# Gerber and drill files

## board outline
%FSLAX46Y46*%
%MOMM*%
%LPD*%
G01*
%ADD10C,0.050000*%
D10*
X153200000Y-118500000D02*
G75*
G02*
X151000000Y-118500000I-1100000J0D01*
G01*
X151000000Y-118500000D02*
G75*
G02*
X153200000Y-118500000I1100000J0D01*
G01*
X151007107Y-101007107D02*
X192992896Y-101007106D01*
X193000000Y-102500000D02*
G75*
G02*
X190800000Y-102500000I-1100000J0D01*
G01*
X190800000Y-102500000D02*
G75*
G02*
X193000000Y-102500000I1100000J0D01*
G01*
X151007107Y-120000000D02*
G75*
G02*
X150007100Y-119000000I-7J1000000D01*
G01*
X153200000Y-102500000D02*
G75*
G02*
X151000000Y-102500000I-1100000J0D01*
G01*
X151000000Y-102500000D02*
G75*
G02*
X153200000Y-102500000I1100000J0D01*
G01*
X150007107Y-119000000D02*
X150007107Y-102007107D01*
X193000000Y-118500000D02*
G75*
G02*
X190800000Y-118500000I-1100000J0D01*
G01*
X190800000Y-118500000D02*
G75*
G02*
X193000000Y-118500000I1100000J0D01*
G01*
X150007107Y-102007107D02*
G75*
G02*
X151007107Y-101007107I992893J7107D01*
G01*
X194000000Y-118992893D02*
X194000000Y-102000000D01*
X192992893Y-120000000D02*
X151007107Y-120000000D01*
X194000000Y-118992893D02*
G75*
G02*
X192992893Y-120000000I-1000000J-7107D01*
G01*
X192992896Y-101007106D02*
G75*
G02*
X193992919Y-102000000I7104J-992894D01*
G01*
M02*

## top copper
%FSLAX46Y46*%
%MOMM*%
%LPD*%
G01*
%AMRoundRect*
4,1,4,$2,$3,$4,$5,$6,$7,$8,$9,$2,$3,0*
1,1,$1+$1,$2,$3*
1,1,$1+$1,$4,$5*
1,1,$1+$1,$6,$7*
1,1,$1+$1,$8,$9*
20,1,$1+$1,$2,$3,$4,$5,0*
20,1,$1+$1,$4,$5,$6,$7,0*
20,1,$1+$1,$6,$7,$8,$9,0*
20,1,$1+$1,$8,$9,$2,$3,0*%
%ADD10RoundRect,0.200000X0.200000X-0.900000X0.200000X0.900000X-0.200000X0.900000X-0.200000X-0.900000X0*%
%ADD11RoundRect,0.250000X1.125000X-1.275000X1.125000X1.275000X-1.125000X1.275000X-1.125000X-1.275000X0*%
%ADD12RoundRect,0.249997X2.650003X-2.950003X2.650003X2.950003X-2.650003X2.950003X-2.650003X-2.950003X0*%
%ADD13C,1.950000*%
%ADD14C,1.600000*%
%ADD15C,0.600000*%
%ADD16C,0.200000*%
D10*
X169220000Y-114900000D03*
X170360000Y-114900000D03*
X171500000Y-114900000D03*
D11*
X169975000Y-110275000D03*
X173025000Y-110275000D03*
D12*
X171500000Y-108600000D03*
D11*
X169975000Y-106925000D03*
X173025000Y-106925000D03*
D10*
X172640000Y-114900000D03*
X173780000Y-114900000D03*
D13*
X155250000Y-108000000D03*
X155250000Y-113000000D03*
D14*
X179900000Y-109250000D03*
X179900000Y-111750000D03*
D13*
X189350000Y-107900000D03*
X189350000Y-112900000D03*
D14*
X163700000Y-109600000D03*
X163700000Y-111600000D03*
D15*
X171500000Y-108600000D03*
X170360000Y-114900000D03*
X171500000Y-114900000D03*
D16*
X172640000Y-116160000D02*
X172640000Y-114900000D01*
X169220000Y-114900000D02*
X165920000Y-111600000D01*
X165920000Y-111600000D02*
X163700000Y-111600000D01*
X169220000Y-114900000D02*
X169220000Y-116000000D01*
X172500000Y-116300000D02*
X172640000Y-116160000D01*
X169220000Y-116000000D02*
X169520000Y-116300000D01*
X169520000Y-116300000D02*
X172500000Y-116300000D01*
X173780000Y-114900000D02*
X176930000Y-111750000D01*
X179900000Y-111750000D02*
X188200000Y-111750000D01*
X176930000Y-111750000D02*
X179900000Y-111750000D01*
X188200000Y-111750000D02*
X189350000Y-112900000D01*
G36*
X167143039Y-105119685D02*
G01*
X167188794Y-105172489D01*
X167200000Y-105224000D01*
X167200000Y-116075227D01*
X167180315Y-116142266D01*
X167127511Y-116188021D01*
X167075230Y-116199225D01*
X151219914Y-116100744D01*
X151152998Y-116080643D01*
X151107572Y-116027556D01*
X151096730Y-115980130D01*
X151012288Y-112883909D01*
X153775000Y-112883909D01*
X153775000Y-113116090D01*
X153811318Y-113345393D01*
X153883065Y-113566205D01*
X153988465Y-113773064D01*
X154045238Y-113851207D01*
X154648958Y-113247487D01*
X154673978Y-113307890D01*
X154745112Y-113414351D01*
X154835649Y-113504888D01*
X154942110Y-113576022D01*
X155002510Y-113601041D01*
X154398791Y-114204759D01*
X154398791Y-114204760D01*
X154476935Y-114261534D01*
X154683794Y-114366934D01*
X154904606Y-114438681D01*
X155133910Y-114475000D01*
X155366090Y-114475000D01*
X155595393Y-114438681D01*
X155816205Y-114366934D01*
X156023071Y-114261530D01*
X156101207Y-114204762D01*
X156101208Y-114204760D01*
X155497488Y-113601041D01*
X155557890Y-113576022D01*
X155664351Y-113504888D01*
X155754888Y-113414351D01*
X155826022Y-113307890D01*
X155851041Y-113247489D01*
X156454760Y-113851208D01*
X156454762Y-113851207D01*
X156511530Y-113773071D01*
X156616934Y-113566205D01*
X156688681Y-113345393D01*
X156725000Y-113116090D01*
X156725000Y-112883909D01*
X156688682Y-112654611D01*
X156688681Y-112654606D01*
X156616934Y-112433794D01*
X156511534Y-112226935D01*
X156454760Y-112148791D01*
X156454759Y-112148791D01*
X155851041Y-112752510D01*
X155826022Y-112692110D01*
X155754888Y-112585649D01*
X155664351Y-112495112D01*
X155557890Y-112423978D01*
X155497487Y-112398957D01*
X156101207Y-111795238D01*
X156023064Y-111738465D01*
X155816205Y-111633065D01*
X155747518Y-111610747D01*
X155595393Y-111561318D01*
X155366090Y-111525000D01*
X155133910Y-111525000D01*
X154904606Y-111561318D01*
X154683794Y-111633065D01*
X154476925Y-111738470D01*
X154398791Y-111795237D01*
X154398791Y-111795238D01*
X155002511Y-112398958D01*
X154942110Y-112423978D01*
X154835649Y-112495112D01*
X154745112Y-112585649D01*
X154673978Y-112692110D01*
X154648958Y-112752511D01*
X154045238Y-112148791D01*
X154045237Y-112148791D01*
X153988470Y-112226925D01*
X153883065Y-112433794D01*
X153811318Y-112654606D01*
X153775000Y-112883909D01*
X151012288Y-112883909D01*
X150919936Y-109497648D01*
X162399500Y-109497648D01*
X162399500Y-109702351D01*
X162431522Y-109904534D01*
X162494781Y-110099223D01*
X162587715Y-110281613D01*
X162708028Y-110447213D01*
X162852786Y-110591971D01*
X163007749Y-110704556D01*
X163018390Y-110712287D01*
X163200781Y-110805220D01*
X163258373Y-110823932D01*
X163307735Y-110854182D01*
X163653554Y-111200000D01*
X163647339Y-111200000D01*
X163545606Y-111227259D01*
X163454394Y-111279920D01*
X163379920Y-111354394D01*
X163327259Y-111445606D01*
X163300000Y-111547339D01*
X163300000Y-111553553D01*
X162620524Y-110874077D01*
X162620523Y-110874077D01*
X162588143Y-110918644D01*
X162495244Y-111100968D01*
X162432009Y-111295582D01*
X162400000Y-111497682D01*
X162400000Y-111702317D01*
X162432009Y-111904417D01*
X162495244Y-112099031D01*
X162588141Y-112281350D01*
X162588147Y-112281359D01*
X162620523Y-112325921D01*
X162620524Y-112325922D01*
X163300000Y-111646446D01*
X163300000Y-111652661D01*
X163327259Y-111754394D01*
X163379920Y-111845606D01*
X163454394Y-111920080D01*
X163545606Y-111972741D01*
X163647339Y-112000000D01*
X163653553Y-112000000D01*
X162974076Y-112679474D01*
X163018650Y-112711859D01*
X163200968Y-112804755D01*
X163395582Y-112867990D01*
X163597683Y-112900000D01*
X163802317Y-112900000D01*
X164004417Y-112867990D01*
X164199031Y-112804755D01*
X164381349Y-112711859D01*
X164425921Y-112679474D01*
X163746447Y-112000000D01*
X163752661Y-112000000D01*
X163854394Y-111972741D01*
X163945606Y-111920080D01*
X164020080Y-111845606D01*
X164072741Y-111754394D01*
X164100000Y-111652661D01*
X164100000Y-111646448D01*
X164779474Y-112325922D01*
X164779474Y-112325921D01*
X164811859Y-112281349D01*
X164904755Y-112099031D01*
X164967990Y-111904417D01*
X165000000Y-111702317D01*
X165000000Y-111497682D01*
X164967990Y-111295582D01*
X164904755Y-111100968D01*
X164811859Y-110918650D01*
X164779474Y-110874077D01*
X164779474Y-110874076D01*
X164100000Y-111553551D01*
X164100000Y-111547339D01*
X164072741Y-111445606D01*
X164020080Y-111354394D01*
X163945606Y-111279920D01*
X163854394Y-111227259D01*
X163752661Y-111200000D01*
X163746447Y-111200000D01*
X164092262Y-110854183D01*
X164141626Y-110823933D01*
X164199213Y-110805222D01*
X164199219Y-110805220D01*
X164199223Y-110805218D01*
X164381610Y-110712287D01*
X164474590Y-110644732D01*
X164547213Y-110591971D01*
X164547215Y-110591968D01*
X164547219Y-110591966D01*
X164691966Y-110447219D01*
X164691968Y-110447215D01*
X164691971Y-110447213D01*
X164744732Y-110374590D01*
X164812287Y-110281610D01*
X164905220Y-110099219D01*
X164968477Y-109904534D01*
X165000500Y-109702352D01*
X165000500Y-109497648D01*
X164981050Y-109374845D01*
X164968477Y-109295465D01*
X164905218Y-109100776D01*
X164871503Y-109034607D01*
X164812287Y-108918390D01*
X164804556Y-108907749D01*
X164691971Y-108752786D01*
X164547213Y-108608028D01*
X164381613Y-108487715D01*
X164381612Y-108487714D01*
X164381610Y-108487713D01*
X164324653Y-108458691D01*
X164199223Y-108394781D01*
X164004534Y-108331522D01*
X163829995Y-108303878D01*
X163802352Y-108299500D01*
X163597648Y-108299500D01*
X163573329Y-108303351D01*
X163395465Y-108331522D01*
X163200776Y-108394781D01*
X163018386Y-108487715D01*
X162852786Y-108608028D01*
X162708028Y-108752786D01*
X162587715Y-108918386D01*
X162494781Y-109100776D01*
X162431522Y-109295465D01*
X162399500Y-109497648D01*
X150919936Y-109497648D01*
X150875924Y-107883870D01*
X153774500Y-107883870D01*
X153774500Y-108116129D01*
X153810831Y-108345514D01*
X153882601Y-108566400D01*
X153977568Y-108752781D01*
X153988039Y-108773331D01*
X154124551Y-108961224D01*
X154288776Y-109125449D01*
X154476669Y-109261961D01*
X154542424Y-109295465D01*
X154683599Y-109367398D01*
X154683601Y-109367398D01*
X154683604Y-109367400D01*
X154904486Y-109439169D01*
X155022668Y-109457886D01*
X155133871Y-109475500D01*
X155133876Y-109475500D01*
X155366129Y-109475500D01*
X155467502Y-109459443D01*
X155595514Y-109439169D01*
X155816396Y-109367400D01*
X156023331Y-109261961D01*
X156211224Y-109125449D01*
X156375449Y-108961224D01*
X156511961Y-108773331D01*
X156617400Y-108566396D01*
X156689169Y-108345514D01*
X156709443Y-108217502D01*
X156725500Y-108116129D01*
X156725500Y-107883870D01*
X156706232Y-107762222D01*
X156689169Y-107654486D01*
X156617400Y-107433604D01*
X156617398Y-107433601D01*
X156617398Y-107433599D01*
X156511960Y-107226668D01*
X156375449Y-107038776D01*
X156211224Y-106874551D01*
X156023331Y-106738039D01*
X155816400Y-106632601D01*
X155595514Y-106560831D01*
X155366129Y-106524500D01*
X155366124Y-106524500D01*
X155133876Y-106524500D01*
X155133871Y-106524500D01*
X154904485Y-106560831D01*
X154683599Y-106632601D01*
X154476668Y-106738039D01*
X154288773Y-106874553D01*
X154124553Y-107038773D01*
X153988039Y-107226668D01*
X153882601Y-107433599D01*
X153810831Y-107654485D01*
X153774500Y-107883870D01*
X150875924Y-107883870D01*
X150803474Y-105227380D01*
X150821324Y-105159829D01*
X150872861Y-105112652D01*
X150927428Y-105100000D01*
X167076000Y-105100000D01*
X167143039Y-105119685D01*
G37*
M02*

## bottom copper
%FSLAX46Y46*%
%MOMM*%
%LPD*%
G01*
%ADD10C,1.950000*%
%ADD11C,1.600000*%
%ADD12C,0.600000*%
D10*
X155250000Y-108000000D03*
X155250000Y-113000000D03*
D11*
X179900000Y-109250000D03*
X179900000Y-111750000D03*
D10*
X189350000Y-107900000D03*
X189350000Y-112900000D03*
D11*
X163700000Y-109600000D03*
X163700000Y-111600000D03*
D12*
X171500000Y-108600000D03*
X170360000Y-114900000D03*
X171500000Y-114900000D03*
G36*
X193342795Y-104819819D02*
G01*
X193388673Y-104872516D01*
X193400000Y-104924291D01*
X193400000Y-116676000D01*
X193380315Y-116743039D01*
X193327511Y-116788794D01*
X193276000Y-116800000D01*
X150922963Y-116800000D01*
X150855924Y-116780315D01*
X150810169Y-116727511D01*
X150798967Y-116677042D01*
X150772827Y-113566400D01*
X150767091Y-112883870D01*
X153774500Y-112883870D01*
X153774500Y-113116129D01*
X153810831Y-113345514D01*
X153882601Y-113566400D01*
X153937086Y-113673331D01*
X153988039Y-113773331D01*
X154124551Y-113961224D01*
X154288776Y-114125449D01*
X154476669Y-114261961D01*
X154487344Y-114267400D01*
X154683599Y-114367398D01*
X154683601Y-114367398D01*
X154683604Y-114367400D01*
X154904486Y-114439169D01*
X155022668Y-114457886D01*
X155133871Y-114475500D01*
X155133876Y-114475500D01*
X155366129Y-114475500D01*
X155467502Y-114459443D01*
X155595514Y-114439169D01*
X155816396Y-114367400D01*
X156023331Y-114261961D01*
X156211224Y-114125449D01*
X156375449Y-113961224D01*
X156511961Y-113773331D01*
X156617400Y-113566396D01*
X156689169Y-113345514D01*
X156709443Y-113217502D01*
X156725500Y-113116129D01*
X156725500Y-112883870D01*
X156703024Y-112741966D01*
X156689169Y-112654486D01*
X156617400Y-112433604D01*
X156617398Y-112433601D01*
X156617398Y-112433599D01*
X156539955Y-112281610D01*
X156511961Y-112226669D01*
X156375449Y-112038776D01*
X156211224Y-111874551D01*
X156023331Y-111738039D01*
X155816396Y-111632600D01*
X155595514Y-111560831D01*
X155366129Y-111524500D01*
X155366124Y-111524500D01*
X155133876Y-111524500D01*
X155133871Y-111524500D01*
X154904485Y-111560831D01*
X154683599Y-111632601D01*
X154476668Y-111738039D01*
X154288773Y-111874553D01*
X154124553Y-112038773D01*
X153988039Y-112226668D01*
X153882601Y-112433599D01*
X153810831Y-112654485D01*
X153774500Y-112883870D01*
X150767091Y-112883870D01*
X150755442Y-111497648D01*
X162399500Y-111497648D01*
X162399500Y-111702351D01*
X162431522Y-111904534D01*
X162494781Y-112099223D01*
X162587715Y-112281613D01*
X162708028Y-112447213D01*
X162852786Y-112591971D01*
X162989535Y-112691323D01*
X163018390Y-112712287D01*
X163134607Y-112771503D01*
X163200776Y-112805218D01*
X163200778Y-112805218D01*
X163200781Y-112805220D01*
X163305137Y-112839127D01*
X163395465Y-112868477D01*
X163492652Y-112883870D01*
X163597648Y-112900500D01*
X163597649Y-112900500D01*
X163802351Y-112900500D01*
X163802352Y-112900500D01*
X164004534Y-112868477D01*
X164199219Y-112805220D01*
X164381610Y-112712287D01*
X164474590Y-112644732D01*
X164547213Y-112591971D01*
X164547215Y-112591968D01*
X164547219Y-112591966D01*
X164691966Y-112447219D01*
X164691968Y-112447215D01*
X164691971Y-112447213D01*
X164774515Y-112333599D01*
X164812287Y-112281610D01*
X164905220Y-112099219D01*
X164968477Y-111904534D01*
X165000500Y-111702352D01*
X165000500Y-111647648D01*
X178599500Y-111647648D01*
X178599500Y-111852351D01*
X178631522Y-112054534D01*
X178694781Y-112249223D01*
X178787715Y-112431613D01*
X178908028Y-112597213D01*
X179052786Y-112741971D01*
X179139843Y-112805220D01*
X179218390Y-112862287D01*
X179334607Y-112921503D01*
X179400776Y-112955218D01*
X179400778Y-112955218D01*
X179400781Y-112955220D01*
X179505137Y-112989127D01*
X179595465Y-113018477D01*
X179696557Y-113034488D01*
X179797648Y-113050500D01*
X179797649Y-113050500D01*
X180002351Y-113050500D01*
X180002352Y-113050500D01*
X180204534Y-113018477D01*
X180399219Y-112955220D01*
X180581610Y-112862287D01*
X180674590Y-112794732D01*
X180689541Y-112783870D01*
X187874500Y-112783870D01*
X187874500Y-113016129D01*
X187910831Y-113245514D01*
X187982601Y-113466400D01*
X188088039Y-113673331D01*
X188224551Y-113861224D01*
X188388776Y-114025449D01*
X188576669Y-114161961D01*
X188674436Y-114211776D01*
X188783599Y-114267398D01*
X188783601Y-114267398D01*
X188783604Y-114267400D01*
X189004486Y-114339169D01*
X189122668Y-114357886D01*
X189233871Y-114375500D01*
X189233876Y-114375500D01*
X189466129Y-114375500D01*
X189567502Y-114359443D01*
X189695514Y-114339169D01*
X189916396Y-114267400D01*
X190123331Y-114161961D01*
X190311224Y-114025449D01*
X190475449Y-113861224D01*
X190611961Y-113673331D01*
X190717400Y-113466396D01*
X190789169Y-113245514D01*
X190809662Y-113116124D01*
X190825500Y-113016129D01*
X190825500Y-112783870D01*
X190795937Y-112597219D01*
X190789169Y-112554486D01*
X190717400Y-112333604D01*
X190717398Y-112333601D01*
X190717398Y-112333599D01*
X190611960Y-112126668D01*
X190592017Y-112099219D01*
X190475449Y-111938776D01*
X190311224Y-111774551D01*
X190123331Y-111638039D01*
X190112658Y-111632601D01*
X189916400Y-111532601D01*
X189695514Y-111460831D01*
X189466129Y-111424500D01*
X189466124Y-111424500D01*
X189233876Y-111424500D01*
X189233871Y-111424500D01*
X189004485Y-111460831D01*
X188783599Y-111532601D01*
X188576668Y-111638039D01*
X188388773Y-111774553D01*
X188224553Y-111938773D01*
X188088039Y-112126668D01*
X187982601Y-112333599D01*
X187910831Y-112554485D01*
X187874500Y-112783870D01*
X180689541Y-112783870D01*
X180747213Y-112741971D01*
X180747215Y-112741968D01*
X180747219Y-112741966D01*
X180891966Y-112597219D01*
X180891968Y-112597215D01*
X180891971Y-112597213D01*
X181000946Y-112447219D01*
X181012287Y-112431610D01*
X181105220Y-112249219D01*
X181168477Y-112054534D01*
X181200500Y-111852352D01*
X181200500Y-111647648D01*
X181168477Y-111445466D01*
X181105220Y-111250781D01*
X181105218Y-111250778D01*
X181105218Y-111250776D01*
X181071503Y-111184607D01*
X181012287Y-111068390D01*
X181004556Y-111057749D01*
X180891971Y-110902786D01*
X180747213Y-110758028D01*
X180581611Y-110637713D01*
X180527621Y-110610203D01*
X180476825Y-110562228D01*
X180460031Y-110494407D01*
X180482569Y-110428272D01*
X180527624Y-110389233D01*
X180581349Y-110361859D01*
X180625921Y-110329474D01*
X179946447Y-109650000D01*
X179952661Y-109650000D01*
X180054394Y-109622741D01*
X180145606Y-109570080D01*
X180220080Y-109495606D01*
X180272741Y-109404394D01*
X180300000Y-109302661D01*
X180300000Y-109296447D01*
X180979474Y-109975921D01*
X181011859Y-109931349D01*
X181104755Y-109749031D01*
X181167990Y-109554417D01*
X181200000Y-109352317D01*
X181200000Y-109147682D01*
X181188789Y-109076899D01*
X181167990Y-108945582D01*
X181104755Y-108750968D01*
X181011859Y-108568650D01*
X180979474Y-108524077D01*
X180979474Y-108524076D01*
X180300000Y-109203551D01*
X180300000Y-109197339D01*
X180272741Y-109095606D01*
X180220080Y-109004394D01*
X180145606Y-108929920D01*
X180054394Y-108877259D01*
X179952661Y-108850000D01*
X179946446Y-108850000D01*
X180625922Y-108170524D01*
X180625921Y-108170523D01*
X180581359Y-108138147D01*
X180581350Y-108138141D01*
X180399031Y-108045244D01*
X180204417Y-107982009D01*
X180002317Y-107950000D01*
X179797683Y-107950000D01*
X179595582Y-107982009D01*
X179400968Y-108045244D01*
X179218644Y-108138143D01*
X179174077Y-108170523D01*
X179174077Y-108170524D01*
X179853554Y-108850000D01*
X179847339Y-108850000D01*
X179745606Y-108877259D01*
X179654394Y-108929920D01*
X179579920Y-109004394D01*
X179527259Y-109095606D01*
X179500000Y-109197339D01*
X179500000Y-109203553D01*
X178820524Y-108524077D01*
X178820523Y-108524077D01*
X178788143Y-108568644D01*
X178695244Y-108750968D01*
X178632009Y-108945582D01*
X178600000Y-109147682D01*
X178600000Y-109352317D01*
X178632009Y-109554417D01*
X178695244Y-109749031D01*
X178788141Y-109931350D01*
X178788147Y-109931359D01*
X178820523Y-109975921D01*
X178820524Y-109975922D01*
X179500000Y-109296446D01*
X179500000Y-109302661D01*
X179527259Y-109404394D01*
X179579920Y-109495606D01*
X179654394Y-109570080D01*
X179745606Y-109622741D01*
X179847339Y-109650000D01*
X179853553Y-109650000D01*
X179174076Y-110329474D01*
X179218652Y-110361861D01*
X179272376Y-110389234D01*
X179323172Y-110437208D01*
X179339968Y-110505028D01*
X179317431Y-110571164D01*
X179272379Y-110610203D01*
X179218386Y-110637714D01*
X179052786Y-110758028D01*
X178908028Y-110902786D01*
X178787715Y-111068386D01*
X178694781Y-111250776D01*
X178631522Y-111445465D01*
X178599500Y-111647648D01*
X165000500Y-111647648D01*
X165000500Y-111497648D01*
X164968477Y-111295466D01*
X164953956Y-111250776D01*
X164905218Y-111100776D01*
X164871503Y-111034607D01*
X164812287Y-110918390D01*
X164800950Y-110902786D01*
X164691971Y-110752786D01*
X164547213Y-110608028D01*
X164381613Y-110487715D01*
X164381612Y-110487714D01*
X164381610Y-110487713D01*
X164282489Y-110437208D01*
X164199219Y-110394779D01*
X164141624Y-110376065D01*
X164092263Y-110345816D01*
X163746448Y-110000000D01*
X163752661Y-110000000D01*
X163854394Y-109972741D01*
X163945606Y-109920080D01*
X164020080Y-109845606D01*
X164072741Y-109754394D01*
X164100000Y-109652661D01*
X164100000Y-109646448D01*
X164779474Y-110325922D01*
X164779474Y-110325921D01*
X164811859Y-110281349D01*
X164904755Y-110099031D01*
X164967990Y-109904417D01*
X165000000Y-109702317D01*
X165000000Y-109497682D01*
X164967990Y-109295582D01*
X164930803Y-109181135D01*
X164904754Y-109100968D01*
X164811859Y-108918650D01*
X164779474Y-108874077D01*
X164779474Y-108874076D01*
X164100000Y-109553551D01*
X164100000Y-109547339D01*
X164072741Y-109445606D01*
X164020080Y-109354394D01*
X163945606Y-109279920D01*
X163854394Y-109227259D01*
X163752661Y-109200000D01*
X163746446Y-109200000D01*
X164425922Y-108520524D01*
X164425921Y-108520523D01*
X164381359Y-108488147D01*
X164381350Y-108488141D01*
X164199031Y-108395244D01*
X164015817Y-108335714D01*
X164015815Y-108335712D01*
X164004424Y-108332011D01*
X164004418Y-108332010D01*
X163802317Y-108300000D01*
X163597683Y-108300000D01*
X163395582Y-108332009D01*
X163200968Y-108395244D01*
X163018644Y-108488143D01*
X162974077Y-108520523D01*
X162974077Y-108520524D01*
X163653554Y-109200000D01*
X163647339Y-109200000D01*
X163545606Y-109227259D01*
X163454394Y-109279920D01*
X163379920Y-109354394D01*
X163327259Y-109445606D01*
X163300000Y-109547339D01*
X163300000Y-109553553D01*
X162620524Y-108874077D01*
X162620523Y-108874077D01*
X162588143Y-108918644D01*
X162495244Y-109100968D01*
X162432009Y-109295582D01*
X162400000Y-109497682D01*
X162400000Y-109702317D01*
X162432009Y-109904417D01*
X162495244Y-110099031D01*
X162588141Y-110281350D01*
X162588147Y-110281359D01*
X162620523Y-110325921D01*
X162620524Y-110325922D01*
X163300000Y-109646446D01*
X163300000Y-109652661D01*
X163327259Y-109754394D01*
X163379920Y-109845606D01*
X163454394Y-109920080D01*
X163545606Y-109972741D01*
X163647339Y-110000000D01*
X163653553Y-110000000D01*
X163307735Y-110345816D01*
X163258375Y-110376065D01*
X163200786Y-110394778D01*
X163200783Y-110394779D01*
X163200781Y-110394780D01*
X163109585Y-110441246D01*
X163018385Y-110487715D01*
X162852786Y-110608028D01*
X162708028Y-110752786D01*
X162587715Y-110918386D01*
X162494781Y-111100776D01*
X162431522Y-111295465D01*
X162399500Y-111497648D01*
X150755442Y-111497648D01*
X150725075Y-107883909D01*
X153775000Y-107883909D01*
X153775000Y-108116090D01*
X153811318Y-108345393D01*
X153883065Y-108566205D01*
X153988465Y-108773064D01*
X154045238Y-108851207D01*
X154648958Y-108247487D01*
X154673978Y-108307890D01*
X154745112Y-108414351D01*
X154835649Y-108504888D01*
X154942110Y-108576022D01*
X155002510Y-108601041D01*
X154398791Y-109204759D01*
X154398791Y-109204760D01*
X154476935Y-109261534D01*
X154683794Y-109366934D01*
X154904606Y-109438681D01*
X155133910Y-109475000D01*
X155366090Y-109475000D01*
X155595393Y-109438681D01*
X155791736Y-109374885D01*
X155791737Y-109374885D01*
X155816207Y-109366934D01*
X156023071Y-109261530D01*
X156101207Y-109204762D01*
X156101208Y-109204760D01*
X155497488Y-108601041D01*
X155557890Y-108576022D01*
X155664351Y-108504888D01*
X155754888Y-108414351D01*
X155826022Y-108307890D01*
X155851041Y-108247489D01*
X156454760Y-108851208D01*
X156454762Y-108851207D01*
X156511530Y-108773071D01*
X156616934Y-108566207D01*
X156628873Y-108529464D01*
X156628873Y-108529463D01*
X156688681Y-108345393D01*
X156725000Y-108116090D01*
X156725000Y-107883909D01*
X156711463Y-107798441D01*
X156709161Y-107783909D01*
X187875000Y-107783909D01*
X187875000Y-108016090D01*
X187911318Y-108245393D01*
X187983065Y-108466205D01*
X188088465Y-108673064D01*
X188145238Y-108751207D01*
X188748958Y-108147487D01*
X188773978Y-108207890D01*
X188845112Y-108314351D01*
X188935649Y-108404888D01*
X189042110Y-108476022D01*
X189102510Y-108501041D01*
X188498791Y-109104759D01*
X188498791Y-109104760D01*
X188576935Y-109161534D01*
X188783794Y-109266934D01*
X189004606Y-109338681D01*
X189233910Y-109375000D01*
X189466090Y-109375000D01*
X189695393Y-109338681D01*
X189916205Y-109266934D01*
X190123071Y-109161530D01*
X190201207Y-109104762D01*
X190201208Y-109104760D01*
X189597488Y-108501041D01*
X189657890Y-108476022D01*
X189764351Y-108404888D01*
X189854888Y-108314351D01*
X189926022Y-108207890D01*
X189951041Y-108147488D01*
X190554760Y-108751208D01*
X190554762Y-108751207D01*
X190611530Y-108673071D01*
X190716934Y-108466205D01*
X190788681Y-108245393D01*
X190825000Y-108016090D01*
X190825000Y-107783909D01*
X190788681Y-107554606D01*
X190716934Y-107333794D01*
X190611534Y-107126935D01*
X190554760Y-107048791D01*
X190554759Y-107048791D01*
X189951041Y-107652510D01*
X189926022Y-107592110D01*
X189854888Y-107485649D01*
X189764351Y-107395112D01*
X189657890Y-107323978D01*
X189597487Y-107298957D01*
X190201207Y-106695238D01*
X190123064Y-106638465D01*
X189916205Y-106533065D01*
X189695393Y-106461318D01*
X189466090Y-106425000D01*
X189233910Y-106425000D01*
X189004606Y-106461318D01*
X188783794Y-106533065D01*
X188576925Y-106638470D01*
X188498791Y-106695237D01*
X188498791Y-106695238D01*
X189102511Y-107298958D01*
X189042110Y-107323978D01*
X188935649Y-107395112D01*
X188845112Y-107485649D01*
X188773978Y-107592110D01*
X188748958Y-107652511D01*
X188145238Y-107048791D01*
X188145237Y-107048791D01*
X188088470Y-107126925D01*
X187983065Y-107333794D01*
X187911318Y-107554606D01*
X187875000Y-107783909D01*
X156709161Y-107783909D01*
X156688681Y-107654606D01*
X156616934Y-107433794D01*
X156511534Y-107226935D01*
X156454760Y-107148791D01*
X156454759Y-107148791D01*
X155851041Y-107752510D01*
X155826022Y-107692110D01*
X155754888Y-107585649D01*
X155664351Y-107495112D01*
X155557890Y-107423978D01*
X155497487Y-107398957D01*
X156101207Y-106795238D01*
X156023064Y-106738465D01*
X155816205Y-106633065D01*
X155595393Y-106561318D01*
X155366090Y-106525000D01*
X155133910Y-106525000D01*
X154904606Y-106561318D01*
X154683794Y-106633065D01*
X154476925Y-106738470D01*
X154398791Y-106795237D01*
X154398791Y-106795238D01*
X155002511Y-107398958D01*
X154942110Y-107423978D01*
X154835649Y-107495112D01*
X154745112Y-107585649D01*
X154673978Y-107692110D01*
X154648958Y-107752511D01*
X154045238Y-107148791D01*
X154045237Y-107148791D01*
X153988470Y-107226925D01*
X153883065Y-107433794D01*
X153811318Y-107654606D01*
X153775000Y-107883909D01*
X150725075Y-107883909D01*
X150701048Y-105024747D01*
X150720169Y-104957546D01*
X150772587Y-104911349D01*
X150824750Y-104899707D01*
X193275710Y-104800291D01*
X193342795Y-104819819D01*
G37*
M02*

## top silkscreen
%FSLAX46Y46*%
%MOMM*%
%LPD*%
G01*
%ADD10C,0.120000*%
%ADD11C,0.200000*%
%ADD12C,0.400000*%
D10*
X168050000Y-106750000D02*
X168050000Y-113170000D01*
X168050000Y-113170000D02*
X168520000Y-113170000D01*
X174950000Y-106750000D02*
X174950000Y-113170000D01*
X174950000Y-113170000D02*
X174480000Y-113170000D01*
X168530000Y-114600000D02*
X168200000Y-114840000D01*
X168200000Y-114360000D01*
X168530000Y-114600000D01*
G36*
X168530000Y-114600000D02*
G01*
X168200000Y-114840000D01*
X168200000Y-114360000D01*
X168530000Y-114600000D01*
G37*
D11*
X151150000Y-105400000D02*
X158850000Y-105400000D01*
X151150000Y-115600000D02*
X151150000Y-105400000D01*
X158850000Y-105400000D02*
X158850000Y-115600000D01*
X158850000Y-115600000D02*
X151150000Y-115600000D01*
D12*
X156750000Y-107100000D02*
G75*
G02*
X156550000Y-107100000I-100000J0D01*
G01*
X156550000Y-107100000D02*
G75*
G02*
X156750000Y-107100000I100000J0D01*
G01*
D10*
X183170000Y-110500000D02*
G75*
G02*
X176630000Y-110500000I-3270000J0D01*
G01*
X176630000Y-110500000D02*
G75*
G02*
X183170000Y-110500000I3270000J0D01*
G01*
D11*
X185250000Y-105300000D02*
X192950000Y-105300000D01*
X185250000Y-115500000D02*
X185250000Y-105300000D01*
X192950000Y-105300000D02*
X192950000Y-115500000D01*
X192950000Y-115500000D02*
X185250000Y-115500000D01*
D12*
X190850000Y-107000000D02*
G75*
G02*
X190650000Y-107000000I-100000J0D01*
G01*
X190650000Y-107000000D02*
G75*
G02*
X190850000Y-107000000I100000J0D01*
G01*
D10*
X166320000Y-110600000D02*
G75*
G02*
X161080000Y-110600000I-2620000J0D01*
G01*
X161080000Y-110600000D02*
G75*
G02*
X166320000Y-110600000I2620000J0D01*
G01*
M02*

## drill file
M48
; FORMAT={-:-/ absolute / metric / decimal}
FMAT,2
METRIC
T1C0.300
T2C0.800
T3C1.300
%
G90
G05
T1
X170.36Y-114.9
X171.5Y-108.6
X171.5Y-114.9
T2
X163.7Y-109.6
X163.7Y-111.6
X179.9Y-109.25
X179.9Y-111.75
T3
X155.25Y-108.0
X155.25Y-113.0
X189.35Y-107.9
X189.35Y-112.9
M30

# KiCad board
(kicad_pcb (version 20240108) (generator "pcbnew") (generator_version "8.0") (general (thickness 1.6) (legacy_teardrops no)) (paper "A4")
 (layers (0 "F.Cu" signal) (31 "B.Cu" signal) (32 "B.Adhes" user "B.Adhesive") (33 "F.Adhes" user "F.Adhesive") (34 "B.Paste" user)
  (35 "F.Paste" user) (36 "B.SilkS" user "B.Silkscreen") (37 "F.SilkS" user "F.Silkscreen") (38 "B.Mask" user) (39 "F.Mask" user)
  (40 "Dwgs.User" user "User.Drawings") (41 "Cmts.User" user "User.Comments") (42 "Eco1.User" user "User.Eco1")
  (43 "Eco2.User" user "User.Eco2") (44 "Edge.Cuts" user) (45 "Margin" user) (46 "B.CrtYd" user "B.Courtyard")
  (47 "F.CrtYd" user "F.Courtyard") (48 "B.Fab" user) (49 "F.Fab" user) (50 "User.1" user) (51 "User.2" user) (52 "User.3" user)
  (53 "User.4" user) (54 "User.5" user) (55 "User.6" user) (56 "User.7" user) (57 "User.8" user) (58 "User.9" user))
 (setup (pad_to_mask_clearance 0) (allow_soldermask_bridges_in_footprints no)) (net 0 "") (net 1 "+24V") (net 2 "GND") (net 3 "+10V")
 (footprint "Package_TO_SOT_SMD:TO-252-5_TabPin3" (layer "F.Cu") (at 171.5 109.86 90)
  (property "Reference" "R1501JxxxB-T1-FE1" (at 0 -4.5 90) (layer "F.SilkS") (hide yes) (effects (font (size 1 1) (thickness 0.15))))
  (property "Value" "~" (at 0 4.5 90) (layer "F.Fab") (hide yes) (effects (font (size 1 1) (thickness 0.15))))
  (fp_line (start 3.11 -3.45) (end -3.31 -3.45) (stroke (width 0.12) (type solid)) (layer "F.SilkS"))
  (fp_line (start -3.31 -3.45) (end -3.31 -2.98) (stroke (width 0.12) (type solid)) (layer "F.SilkS"))
  (fp_line (start 3.11 3.45) (end -3.31 3.45) (stroke (width 0.12) (type solid)) (layer "F.SilkS"))
  (fp_line (start -3.31 3.45) (end -3.31 2.98) (stroke (width 0.12) (type solid)) (layer "F.SilkS"))
  (fp_poly
   (pts (xy -4.74 -2.97) (xy -4.98 -3.3) (xy -4.5 -3.3) (xy -4.74 -2.97)) (stroke (width 0.12) (type solid)) (fill solid) (layer "F.SilkS"))
  (pad "1" smd roundrect (at -5.04 -2.28 90) (size 2.2 0.8) (layers "F.Cu" "F.Paste" "F.Mask") (roundrect_rratio 0.25) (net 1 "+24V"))
  (pad "2" smd roundrect (at -5.04 -1.14 90) (size 2.2 0.8) (layers "F.Cu" "F.Paste" "F.Mask") (roundrect_rratio 0.25) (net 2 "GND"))
  (pad "3" smd roundrect (at -5.04 0 90) (size 2.2 0.8) (layers "F.Cu" "F.Paste" "F.Mask") (roundrect_rratio 0.25) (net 2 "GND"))
  (pad "3" smd roundrect (at -0.415 -1.525 90) (size 3.05 2.75) (layers "F.Cu" "F.Paste") (roundrect_rratio 0.090909) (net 2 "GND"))
  (pad "3" smd roundrect (at -0.415 1.525 90) (size 3.05 2.75) (layers "F.Cu" "F.Paste") (roundrect_rratio 0.090909) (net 2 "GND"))
  (pad "3" smd roundrect (at 1.26 0 90) (size 6.4 5.8) (layers "F.Cu" "F.Mask") (roundrect_rratio 0.043103) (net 2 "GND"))
  (pad "3" smd roundrect (at 2.935 -1.525 90) (size 3.05 2.75) (layers "F.Cu" "F.Paste") (roundrect_rratio 0.090909) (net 2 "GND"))
  (pad "3" smd roundrect (at 2.935 1.525 90) (size 3.05 2.75) (layers "F.Cu" "F.Paste") (roundrect_rratio 0.090909) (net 2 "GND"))
  (pad "4" smd roundrect (at -5.04 1.14 90) (size 2.2 0.8) (layers "F.Cu" "F.Paste" "F.Mask") (roundrect_rratio 0.25) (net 1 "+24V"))
  (pad "5" smd roundrect (at -5.04 2.28 90) (size 2.2 0.8) (layers "F.Cu" "F.Paste" "F.Mask") (roundrect_rratio 0.25) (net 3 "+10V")))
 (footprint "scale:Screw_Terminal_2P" (layer "F.Cu") (at 155.25 110.5 -90)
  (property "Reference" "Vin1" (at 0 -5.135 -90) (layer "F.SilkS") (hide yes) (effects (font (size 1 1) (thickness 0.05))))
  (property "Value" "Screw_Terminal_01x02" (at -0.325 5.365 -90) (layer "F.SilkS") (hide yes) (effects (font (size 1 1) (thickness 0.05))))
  (fp_line (start -5.1 4.1) (end -5.1 -3.6) (stroke (width 0.2) (type solid)) (layer "F.SilkS"))
  (fp_line (start 5.1 4.1) (end -5.1 4.1) (stroke (width 0.2) (type solid)) (layer "F.SilkS"))
  (fp_line (start -5.1 -3.6) (end 5.1 -3.6) (stroke (width 0.2) (type solid)) (layer "F.SilkS"))
  (fp_line (start 5.1 -3.6) (end 5.1 4.1) (stroke (width 0.2) (type solid)) (layer "F.SilkS"))
  (fp_circle (center -3.4 -1.4) (end -3.3 -1.4) (stroke (width 0.4) (type solid)) (fill none) (layer "F.SilkS"))
  (pad "1" thru_hole circle (at -2.5 0 270) (size 1.95 1.95) (drill 1.3) (layers "*.Cu" "*.Mask") (remove_unused_layers no) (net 2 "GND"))
  (pad "2" thru_hole circle (at 2.5 0 270) (size 1.95 1.95) (drill 1.3) (layers "*.Cu" "*.Mask") (remove_unused_layers no) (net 1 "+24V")))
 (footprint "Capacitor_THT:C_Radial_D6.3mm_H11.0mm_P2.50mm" (layer "F.Cu") (at 179.9 109.25 -90)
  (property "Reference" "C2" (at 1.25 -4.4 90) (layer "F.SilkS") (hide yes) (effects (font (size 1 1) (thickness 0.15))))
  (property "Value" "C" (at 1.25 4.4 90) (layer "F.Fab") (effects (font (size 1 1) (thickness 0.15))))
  (fp_circle (center 1.25 0) (end 4.52 0) (stroke (width 0.12) (type solid)) (fill none) (layer "F.SilkS"))
  (pad "1" thru_hole circle (at 0 0 270) (size 1.6 1.6) (drill 0.8) (layers "*.Cu" "*.Mask") (remove_unused_layers no) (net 2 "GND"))
  (pad "2" thru_hole circle (at 2.5 0 270) (size 1.6 1.6) (drill 0.8) (layers "*.Cu" "*.Mask") (remove_unused_layers no) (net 3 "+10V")))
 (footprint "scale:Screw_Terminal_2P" (layer "F.Cu") (at 189.35 110.4 -90)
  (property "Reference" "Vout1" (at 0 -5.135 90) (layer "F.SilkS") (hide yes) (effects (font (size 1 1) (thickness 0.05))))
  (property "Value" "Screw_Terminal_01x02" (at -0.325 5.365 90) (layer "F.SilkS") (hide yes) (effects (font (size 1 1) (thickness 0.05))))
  (fp_line (start -5.1 4.1) (end -5.1 -3.6) (stroke (width 0.2) (type solid)) (layer "F.SilkS"))
  (fp_line (start 5.1 4.1) (end -5.1 4.1) (stroke (width 0.2) (type solid)) (layer "F.SilkS"))
  (fp_line (start -5.1 -3.6) (end 5.1 -3.6) (stroke (width 0.2) (type solid)) (layer "F.SilkS"))
  (fp_line (start 5.1 -3.6) (end 5.1 4.1) (stroke (width 0.2) (type solid)) (layer "F.SilkS"))
  (fp_circle (center -3.4 -1.4) (end -3.3 -1.4) (stroke (width 0.4) (type solid)) (fill none) (layer "F.SilkS"))
  (pad "1" thru_hole circle (at -2.5 0 270) (size 1.95 1.95) (drill 1.3) (layers "*.Cu" "*.Mask") (remove_unused_layers no) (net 2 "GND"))
  (pad "2" thru_hole circle (at 2.5 0 270) (size 1.95 1.95) (drill 1.3) (layers "*.Cu" "*.Mask") (remove_unused_layers no) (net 3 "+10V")))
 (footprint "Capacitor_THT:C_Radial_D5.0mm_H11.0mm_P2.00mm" (layer "F.Cu") (at 163.7 109.6 -90)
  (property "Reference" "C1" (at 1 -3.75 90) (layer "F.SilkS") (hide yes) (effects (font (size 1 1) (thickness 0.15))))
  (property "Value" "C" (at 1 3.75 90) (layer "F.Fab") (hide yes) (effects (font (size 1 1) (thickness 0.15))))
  (fp_circle (center 1 0) (end 3.62 0) (stroke (width 0.12) (type solid)) (fill none) (layer "F.SilkS"))
  (pad "1" thru_hole circle (at 0 0 270) (size 1.6 1.6) (drill 0.8) (layers "*.Cu" "*.Mask") (remove_unused_layers no) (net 2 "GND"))
  (pad "2" thru_hole circle (at 2 0 270) (size 1.6 1.6) (drill 0.8) (layers "*.Cu" "*.Mask") (remove_unused_layers no) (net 1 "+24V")))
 (gr_circle (center 152.1 118.5) (end 153.2 118.5) (stroke (width 0.05) (type default)) (fill none) (layer "Edge.Cuts"))
 (gr_line (start 151.007107 101.007107) (end 192.992896 101.007106) (stroke (width 0.05) (type default)) (layer "Edge.Cuts"))
 (gr_circle (center 191.9 102.5) (end 193 102.5) (stroke (width 0.05) (type default)) (fill none) (layer "Edge.Cuts"))
 (gr_arc (start 151.007107 120) (mid 150.3 119.707107) (end 150.007107 119) (stroke (width 0.05) (type default)) (layer "Edge.Cuts"))
 (gr_circle (center 152.1 102.5) (end 153.2 102.5) (stroke (width 0.05) (type default)) (fill none) (layer "Edge.Cuts"))
 (gr_line (start 150.007107 119) (end 150.007107 102.007107) (stroke (width 0.05) (type default)) (layer "Edge.Cuts"))
 (gr_circle (center 191.9 118.5) (end 193 118.5) (stroke (width 0.05) (type default)) (fill none) (layer "Edge.Cuts"))
 (gr_arc (start 150.007107 102.007107) (mid 150.297901 101.297901) (end 151.007107 101.007107) (stroke (width 0.05) (type default))
  (layer "Edge.Cuts"))
 (gr_line (start 194 118.992893) (end 194 102) (stroke (width 0.05) (type default)) (layer "Edge.Cuts"))
 (gr_line (start 192.992893 120) (end 151.007107 120) (stroke (width 0.05) (type default)) (layer "Edge.Cuts"))
 (gr_arc (start 194 118.992893) (mid 193.707125 119.707125) (end 192.992893 120) (stroke (width 0.05) (type default)) (layer "Edge.Cuts"))
 (gr_arc (start 192.992896 101.007106) (mid 193.699584 101.295393) (end 193.992919 102) (stroke (width 0.05) (type default))
  (layer "Edge.Cuts"))
 (via (at 171.5 108.6) (size 0.6) (drill 0.3) (layers "F.Cu" "B.Cu") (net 2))
 (via (at 170.36 114.9) (size 0.6) (drill 0.3) (layers "F.Cu" "B.Cu") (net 2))
 (via (at 171.5 114.9) (size 0.6) (drill 0.3) (layers "F.Cu" "B.Cu") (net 2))
 (segment (start 172.64 116.16) (end 172.64 114.9) (width 0.2) (layer "F.Cu") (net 1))
 (segment (start 169.22 114.9) (end 165.92 111.6) (width 0.2) (layer "F.Cu") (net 1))
 (segment (start 165.92 111.6) (end 163.7 111.6) (width 0.2) (layer "F.Cu") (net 1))
 (segment (start 169.22 114.9) (end 169.22 116) (width 0.2) (layer "F.Cu") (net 1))
 (segment (start 172.5 116.3) (end 172.64 116.16) (width 0.2) (layer "F.Cu") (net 1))
 (segment (start 169.22 116) (end 169.52 116.3) (width 0.2) (layer "F.Cu") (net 1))
 (segment (start 169.52 116.3) (end 172.5 116.3) (width 0.2) (layer "F.Cu") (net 1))
 (segment (start 173.78 114.9) (end 176.93 111.75) (width 0.2) (layer "F.Cu") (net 3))
 (segment (start 179.9 111.75) (end 188.2 111.75) (width 0.2) (layer "F.Cu") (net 3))
 (segment (start 176.93 111.75) (end 179.9 111.75) (width 0.2) (layer "F.Cu") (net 3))
 (segment (start 188.2 111.75) (end 189.35 112.9) (width 0.2) (layer "F.Cu") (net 3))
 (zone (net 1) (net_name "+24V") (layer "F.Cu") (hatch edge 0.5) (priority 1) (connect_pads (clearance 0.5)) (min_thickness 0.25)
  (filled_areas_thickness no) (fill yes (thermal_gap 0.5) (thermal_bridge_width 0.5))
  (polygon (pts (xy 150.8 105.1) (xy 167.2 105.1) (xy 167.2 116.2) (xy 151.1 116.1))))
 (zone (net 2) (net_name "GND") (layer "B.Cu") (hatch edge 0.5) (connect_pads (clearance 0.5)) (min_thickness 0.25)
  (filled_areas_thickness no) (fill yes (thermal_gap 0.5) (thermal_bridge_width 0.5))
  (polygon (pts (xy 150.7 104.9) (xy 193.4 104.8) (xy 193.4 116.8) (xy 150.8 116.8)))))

